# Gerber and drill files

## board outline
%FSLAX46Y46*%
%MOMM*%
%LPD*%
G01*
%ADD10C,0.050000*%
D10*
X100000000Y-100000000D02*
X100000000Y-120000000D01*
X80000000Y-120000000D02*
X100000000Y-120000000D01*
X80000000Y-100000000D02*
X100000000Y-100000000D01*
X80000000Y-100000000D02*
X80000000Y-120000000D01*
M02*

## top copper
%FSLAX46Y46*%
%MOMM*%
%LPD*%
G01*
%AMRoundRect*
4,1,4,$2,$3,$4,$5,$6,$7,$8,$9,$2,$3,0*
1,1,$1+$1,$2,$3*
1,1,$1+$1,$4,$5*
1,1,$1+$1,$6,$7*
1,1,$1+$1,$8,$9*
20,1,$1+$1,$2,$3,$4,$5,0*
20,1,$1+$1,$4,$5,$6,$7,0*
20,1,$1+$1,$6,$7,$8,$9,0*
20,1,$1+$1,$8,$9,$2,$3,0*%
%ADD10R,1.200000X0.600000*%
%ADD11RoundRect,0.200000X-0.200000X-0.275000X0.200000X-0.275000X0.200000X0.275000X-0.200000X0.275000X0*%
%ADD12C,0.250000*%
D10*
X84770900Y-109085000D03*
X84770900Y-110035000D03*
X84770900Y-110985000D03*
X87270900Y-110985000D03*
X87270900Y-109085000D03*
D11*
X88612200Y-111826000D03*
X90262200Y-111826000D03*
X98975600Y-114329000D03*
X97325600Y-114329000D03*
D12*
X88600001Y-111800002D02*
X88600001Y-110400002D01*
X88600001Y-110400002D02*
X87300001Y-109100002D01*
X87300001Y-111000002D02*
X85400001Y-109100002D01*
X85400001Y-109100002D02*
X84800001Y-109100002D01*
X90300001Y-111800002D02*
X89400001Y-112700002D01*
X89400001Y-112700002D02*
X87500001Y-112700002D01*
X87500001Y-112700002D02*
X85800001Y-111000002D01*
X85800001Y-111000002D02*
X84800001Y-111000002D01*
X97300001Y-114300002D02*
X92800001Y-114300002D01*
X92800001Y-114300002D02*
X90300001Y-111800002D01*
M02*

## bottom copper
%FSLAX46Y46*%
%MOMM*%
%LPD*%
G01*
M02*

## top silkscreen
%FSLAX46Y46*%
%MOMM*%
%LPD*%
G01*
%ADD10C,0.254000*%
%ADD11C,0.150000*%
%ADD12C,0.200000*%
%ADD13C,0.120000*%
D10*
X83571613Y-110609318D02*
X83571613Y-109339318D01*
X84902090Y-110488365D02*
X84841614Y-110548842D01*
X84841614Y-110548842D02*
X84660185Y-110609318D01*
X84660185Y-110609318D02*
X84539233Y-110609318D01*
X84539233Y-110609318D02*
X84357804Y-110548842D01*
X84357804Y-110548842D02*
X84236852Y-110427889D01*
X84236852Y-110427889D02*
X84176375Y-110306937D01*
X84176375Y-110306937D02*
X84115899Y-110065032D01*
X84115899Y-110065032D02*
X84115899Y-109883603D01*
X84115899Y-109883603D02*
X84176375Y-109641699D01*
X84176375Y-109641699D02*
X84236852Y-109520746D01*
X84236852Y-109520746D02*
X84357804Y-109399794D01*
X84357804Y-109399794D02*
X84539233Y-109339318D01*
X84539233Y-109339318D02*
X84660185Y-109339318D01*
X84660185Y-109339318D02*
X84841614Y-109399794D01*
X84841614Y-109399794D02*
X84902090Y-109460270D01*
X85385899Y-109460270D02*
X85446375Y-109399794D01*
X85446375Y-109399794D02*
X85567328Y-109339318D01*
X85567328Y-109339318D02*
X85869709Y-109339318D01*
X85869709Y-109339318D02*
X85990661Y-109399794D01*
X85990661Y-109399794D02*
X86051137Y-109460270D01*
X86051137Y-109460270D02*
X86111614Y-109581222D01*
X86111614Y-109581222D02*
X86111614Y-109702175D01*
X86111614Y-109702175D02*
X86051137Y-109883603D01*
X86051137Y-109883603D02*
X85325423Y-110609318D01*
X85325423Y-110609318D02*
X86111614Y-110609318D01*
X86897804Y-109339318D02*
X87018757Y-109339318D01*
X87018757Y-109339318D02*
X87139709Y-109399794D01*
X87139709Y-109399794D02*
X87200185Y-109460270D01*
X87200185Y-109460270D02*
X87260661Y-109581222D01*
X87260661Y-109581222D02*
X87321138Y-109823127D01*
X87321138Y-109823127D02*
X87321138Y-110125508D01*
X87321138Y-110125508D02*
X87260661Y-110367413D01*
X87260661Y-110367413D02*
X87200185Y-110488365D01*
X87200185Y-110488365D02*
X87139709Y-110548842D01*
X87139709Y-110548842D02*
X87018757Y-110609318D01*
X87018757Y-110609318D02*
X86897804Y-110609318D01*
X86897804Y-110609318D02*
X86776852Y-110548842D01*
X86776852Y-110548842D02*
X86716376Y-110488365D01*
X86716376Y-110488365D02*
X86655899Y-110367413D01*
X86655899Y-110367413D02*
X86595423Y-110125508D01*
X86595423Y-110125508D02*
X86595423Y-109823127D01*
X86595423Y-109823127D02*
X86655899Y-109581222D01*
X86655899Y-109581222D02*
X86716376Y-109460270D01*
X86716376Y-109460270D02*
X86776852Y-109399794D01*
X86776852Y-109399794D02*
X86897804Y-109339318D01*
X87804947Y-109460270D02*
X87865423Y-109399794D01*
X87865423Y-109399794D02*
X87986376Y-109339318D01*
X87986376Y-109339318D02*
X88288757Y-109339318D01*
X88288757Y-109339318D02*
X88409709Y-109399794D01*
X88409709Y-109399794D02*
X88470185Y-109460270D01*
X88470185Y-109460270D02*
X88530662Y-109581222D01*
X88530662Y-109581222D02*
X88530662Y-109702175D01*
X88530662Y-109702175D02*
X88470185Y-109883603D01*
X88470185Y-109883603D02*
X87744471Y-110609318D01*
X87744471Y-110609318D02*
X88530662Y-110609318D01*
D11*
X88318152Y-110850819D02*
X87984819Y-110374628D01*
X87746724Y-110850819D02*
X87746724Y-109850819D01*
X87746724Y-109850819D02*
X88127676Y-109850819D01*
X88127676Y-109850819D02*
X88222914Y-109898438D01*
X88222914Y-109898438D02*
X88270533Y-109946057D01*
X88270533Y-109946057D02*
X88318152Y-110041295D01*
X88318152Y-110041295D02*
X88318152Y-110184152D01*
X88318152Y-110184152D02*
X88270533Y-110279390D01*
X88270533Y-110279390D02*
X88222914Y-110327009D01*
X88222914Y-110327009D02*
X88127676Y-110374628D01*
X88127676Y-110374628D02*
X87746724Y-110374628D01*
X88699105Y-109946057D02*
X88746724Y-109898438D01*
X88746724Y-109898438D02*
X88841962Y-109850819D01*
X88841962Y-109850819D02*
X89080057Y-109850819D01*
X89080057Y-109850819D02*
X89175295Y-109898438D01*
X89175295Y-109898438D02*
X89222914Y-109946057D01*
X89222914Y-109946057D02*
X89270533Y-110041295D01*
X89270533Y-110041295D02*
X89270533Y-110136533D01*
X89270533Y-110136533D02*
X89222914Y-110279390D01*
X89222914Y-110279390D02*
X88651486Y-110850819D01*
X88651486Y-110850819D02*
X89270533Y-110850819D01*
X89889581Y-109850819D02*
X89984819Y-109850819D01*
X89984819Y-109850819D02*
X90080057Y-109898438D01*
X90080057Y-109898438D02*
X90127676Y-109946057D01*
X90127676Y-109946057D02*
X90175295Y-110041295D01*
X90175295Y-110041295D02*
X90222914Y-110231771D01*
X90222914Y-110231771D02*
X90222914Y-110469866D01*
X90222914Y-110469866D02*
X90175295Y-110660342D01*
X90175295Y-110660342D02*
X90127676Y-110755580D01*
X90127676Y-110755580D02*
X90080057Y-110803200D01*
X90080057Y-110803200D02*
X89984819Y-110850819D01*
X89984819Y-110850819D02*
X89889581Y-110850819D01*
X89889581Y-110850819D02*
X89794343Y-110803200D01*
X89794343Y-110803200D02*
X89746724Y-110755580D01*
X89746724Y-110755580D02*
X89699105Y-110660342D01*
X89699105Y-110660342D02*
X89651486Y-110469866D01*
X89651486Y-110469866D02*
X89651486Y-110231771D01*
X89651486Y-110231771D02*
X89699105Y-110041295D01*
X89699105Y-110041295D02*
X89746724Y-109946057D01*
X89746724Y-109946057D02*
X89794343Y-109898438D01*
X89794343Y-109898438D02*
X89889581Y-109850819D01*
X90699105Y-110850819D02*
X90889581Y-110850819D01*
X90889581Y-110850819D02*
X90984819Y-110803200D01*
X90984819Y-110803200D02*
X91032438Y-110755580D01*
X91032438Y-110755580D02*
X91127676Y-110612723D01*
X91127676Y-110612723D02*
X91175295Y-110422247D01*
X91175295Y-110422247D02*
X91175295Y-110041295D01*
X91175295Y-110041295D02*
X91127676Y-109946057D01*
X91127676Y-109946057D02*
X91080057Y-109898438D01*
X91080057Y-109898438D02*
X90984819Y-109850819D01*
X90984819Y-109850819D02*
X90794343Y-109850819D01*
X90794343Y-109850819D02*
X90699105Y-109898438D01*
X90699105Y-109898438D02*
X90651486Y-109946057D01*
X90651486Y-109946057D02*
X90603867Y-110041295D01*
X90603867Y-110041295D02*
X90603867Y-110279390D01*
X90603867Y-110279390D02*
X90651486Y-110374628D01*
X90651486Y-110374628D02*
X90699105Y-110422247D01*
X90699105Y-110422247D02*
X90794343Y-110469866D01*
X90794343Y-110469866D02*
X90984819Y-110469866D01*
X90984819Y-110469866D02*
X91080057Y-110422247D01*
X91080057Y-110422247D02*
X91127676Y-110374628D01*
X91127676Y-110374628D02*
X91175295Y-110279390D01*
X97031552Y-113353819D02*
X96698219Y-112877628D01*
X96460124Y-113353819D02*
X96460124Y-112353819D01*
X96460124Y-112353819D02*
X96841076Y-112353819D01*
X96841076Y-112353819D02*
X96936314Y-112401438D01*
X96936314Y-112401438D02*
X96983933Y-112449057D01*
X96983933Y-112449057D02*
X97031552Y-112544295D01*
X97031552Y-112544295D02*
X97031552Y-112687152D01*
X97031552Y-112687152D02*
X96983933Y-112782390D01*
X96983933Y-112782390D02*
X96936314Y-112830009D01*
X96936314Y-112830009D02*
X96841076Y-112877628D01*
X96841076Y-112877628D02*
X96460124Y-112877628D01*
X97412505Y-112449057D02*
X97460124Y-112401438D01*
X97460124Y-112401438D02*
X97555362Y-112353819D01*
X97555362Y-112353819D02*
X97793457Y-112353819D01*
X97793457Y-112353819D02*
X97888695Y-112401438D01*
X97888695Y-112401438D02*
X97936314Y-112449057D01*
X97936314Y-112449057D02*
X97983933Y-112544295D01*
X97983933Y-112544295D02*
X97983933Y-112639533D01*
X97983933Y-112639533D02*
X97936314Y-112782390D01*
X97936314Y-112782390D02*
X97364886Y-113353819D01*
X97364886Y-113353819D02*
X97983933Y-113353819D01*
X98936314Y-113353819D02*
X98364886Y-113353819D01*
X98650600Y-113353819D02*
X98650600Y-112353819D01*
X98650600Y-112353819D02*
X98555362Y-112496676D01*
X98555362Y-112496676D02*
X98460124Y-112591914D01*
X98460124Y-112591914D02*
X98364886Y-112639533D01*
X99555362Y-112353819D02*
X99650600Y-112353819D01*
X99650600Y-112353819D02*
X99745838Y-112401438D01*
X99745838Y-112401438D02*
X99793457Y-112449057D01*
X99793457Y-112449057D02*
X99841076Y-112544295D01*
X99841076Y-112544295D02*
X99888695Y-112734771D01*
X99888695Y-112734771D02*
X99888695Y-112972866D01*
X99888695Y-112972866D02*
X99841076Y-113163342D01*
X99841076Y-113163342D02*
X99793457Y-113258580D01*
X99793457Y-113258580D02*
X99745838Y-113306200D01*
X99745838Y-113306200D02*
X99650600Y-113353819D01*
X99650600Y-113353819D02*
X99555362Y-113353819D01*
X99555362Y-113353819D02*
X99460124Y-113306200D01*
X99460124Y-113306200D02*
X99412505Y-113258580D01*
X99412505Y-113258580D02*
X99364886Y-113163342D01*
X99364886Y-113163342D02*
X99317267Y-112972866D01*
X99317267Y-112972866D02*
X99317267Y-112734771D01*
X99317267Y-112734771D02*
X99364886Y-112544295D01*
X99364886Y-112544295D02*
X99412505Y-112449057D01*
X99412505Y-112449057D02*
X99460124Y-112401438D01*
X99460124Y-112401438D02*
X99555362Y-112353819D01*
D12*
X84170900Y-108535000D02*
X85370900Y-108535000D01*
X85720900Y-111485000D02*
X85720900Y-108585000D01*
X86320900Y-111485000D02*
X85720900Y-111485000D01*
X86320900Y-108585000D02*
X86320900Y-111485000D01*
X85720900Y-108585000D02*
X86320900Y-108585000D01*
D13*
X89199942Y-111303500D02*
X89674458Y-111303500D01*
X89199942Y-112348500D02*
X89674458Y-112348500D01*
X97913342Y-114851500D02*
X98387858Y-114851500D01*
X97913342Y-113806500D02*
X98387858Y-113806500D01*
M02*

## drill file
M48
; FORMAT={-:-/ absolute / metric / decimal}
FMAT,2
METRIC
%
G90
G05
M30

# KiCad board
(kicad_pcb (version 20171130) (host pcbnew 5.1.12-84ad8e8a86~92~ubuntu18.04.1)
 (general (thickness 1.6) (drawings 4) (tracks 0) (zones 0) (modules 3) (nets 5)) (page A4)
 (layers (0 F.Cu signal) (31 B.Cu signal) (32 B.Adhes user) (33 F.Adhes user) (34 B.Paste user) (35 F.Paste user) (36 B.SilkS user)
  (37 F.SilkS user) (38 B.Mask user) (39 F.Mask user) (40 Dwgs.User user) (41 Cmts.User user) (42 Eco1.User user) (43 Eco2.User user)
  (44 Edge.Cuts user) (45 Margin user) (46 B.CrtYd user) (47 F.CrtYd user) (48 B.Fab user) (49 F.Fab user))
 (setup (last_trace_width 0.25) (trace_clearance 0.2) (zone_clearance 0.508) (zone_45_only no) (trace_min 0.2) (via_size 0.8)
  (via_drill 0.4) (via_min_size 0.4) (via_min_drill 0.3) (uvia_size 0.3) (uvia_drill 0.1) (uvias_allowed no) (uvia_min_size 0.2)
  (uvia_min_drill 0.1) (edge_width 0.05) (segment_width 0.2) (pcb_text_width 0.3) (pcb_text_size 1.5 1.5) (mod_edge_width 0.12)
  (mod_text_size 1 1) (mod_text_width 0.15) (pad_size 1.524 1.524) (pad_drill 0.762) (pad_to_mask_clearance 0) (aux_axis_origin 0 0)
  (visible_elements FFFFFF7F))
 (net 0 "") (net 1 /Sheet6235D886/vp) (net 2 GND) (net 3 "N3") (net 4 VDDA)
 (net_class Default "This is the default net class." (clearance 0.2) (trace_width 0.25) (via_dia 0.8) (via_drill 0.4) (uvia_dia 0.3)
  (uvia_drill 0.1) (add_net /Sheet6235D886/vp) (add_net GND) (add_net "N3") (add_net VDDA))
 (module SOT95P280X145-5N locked (layer F.Cu) (at 86.020900 110.035000)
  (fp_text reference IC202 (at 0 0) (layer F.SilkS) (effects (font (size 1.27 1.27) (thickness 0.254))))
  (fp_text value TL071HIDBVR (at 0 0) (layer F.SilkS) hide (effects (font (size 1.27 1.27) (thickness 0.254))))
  (fp_line (start -1.85 -1.5) (end -0.65 -1.5) (layer F.SilkS) (width 0.2))
  (fp_line (start -0.3 1.45) (end -0.3 -1.45) (layer F.SilkS) (width 0.2))
  (fp_line (start 0.3 1.45) (end -0.3 1.45) (layer F.SilkS) (width 0.2))
  (fp_line (start 0.3 -1.45) (end 0.3 1.45) (layer F.SilkS) (width 0.2))
  (fp_line (start -0.3 -1.45) (end 0.3 -1.45) (layer F.SilkS) (width 0.2))
  (pad 1 smd rect (at -1.25 -0.95 90.000000) (size 0.6 1.2) (layers F.Cu F.Mask F.Paste) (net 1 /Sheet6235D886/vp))
  (pad 2 smd rect (at -1.25 0 90.000000) (size 0.6 1.2) (layers F.Cu F.Mask F.Paste) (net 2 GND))
  (pad 3 smd rect (at -1.25 0.95 90.000000) (size 0.6 1.2) (layers F.Cu F.Mask F.Paste) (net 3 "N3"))
  (pad 4 smd rect (at 1.25 0.95 90.000000) (size 0.6 1.2) (layers F.Cu F.Mask F.Paste) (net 1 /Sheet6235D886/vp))
  (pad 5 smd rect (at 1.25 -0.95 90.000000) (size 0.6 1.2) (layers F.Cu F.Mask F.Paste) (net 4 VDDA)))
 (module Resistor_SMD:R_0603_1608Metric (layer F.Cu) (at 89.437200 111.826000)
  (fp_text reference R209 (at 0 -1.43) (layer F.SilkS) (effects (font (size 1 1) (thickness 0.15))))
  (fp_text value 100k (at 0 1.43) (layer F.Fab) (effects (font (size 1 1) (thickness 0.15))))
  (fp_line (start -0.237258 -0.5225) (end 0.237258 -0.5225) (layer F.SilkS) (width 0.12))
  (fp_line (start -0.237258 0.5225) (end 0.237258 0.5225) (layer F.SilkS) (width 0.12))
  (pad 1 smd roundrect (at -0.825 0) (size 0.8 0.95) (layers F.Cu F.Mask F.Paste) (roundrect_rratio 0.25) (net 4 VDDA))
  (pad 2 smd roundrect (at 0.825 0) (size 0.8 0.95) (layers F.Cu F.Mask F.Paste) (roundrect_rratio 0.25) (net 3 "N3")))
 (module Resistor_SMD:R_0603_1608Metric (layer F.Cu) (at 98.150600 114.329000)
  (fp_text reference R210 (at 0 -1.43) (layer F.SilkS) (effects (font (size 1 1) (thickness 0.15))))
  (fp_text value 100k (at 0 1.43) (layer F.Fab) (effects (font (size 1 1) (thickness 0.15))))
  (fp_line (start -0.237258 0.5225) (end 0.237258 0.5225) (layer F.SilkS) (width 0.12))
  (fp_line (start -0.237258 -0.5225) (end 0.237258 -0.5225) (layer F.SilkS) (width 0.12))
  (pad 2 smd roundrect (at 0.825 0) (size 0.8 0.95) (layers F.Cu F.Mask F.Paste) (roundrect_rratio 0.25) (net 2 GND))
  (pad 1 smd roundrect (at -0.825 0) (size 0.8 0.95) (layers F.Cu F.Mask F.Paste) (roundrect_rratio 0.25) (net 3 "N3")))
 (gr_line (start 100 100) (end 100 120) (layer Edge.Cuts) (width 0.05))
 (gr_line (start 80 120) (end 100 120) (layer Edge.Cuts) (width 0.05))
 (gr_line (start 80 100) (end 100 100) (layer Edge.Cuts) (width 0.05))
 (gr_line (start 80 100) (end 80 120) (layer Edge.Cuts) (width 0.05))
 (segment (start 88.600001 111.800002) (end 88.600001 110.400002) (width 0.250000) (layer F.Cu) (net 4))
 (segment (start 88.600001 110.400002) (end 87.300001 109.100002) (width 0.250000) (layer F.Cu) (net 4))
 (segment (start 87.300001 111.000002) (end 85.400001 109.100002) (width 0.250000) (layer F.Cu) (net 1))
 (segment (start 85.400001 109.100002) (end 84.800001 109.100002) (width 0.250000) (layer F.Cu) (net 1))
 (segment (start 90.300001 111.800002) (end 89.400001 112.700002) (width 0.250000) (layer F.Cu) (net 3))
 (segment (start 89.400001 112.700002) (end 87.500001 112.700002) (width 0.250000) (layer F.Cu) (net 3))
 (segment (start 87.500001 112.700002) (end 85.800001 111.000002) (width 0.250000) (layer F.Cu) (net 3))
 (segment (start 85.800001 111.000002) (end 84.800001 111.000002) (width 0.250000) (layer F.Cu) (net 3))
 (segment (start 97.300001 114.300002) (end 92.800001 114.300002) (width 0.250000) (layer F.Cu) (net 3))
 (segment (start 92.800001 114.300002) (end 90.300001 111.800002) (width 0.250000) (layer F.Cu) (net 3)))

